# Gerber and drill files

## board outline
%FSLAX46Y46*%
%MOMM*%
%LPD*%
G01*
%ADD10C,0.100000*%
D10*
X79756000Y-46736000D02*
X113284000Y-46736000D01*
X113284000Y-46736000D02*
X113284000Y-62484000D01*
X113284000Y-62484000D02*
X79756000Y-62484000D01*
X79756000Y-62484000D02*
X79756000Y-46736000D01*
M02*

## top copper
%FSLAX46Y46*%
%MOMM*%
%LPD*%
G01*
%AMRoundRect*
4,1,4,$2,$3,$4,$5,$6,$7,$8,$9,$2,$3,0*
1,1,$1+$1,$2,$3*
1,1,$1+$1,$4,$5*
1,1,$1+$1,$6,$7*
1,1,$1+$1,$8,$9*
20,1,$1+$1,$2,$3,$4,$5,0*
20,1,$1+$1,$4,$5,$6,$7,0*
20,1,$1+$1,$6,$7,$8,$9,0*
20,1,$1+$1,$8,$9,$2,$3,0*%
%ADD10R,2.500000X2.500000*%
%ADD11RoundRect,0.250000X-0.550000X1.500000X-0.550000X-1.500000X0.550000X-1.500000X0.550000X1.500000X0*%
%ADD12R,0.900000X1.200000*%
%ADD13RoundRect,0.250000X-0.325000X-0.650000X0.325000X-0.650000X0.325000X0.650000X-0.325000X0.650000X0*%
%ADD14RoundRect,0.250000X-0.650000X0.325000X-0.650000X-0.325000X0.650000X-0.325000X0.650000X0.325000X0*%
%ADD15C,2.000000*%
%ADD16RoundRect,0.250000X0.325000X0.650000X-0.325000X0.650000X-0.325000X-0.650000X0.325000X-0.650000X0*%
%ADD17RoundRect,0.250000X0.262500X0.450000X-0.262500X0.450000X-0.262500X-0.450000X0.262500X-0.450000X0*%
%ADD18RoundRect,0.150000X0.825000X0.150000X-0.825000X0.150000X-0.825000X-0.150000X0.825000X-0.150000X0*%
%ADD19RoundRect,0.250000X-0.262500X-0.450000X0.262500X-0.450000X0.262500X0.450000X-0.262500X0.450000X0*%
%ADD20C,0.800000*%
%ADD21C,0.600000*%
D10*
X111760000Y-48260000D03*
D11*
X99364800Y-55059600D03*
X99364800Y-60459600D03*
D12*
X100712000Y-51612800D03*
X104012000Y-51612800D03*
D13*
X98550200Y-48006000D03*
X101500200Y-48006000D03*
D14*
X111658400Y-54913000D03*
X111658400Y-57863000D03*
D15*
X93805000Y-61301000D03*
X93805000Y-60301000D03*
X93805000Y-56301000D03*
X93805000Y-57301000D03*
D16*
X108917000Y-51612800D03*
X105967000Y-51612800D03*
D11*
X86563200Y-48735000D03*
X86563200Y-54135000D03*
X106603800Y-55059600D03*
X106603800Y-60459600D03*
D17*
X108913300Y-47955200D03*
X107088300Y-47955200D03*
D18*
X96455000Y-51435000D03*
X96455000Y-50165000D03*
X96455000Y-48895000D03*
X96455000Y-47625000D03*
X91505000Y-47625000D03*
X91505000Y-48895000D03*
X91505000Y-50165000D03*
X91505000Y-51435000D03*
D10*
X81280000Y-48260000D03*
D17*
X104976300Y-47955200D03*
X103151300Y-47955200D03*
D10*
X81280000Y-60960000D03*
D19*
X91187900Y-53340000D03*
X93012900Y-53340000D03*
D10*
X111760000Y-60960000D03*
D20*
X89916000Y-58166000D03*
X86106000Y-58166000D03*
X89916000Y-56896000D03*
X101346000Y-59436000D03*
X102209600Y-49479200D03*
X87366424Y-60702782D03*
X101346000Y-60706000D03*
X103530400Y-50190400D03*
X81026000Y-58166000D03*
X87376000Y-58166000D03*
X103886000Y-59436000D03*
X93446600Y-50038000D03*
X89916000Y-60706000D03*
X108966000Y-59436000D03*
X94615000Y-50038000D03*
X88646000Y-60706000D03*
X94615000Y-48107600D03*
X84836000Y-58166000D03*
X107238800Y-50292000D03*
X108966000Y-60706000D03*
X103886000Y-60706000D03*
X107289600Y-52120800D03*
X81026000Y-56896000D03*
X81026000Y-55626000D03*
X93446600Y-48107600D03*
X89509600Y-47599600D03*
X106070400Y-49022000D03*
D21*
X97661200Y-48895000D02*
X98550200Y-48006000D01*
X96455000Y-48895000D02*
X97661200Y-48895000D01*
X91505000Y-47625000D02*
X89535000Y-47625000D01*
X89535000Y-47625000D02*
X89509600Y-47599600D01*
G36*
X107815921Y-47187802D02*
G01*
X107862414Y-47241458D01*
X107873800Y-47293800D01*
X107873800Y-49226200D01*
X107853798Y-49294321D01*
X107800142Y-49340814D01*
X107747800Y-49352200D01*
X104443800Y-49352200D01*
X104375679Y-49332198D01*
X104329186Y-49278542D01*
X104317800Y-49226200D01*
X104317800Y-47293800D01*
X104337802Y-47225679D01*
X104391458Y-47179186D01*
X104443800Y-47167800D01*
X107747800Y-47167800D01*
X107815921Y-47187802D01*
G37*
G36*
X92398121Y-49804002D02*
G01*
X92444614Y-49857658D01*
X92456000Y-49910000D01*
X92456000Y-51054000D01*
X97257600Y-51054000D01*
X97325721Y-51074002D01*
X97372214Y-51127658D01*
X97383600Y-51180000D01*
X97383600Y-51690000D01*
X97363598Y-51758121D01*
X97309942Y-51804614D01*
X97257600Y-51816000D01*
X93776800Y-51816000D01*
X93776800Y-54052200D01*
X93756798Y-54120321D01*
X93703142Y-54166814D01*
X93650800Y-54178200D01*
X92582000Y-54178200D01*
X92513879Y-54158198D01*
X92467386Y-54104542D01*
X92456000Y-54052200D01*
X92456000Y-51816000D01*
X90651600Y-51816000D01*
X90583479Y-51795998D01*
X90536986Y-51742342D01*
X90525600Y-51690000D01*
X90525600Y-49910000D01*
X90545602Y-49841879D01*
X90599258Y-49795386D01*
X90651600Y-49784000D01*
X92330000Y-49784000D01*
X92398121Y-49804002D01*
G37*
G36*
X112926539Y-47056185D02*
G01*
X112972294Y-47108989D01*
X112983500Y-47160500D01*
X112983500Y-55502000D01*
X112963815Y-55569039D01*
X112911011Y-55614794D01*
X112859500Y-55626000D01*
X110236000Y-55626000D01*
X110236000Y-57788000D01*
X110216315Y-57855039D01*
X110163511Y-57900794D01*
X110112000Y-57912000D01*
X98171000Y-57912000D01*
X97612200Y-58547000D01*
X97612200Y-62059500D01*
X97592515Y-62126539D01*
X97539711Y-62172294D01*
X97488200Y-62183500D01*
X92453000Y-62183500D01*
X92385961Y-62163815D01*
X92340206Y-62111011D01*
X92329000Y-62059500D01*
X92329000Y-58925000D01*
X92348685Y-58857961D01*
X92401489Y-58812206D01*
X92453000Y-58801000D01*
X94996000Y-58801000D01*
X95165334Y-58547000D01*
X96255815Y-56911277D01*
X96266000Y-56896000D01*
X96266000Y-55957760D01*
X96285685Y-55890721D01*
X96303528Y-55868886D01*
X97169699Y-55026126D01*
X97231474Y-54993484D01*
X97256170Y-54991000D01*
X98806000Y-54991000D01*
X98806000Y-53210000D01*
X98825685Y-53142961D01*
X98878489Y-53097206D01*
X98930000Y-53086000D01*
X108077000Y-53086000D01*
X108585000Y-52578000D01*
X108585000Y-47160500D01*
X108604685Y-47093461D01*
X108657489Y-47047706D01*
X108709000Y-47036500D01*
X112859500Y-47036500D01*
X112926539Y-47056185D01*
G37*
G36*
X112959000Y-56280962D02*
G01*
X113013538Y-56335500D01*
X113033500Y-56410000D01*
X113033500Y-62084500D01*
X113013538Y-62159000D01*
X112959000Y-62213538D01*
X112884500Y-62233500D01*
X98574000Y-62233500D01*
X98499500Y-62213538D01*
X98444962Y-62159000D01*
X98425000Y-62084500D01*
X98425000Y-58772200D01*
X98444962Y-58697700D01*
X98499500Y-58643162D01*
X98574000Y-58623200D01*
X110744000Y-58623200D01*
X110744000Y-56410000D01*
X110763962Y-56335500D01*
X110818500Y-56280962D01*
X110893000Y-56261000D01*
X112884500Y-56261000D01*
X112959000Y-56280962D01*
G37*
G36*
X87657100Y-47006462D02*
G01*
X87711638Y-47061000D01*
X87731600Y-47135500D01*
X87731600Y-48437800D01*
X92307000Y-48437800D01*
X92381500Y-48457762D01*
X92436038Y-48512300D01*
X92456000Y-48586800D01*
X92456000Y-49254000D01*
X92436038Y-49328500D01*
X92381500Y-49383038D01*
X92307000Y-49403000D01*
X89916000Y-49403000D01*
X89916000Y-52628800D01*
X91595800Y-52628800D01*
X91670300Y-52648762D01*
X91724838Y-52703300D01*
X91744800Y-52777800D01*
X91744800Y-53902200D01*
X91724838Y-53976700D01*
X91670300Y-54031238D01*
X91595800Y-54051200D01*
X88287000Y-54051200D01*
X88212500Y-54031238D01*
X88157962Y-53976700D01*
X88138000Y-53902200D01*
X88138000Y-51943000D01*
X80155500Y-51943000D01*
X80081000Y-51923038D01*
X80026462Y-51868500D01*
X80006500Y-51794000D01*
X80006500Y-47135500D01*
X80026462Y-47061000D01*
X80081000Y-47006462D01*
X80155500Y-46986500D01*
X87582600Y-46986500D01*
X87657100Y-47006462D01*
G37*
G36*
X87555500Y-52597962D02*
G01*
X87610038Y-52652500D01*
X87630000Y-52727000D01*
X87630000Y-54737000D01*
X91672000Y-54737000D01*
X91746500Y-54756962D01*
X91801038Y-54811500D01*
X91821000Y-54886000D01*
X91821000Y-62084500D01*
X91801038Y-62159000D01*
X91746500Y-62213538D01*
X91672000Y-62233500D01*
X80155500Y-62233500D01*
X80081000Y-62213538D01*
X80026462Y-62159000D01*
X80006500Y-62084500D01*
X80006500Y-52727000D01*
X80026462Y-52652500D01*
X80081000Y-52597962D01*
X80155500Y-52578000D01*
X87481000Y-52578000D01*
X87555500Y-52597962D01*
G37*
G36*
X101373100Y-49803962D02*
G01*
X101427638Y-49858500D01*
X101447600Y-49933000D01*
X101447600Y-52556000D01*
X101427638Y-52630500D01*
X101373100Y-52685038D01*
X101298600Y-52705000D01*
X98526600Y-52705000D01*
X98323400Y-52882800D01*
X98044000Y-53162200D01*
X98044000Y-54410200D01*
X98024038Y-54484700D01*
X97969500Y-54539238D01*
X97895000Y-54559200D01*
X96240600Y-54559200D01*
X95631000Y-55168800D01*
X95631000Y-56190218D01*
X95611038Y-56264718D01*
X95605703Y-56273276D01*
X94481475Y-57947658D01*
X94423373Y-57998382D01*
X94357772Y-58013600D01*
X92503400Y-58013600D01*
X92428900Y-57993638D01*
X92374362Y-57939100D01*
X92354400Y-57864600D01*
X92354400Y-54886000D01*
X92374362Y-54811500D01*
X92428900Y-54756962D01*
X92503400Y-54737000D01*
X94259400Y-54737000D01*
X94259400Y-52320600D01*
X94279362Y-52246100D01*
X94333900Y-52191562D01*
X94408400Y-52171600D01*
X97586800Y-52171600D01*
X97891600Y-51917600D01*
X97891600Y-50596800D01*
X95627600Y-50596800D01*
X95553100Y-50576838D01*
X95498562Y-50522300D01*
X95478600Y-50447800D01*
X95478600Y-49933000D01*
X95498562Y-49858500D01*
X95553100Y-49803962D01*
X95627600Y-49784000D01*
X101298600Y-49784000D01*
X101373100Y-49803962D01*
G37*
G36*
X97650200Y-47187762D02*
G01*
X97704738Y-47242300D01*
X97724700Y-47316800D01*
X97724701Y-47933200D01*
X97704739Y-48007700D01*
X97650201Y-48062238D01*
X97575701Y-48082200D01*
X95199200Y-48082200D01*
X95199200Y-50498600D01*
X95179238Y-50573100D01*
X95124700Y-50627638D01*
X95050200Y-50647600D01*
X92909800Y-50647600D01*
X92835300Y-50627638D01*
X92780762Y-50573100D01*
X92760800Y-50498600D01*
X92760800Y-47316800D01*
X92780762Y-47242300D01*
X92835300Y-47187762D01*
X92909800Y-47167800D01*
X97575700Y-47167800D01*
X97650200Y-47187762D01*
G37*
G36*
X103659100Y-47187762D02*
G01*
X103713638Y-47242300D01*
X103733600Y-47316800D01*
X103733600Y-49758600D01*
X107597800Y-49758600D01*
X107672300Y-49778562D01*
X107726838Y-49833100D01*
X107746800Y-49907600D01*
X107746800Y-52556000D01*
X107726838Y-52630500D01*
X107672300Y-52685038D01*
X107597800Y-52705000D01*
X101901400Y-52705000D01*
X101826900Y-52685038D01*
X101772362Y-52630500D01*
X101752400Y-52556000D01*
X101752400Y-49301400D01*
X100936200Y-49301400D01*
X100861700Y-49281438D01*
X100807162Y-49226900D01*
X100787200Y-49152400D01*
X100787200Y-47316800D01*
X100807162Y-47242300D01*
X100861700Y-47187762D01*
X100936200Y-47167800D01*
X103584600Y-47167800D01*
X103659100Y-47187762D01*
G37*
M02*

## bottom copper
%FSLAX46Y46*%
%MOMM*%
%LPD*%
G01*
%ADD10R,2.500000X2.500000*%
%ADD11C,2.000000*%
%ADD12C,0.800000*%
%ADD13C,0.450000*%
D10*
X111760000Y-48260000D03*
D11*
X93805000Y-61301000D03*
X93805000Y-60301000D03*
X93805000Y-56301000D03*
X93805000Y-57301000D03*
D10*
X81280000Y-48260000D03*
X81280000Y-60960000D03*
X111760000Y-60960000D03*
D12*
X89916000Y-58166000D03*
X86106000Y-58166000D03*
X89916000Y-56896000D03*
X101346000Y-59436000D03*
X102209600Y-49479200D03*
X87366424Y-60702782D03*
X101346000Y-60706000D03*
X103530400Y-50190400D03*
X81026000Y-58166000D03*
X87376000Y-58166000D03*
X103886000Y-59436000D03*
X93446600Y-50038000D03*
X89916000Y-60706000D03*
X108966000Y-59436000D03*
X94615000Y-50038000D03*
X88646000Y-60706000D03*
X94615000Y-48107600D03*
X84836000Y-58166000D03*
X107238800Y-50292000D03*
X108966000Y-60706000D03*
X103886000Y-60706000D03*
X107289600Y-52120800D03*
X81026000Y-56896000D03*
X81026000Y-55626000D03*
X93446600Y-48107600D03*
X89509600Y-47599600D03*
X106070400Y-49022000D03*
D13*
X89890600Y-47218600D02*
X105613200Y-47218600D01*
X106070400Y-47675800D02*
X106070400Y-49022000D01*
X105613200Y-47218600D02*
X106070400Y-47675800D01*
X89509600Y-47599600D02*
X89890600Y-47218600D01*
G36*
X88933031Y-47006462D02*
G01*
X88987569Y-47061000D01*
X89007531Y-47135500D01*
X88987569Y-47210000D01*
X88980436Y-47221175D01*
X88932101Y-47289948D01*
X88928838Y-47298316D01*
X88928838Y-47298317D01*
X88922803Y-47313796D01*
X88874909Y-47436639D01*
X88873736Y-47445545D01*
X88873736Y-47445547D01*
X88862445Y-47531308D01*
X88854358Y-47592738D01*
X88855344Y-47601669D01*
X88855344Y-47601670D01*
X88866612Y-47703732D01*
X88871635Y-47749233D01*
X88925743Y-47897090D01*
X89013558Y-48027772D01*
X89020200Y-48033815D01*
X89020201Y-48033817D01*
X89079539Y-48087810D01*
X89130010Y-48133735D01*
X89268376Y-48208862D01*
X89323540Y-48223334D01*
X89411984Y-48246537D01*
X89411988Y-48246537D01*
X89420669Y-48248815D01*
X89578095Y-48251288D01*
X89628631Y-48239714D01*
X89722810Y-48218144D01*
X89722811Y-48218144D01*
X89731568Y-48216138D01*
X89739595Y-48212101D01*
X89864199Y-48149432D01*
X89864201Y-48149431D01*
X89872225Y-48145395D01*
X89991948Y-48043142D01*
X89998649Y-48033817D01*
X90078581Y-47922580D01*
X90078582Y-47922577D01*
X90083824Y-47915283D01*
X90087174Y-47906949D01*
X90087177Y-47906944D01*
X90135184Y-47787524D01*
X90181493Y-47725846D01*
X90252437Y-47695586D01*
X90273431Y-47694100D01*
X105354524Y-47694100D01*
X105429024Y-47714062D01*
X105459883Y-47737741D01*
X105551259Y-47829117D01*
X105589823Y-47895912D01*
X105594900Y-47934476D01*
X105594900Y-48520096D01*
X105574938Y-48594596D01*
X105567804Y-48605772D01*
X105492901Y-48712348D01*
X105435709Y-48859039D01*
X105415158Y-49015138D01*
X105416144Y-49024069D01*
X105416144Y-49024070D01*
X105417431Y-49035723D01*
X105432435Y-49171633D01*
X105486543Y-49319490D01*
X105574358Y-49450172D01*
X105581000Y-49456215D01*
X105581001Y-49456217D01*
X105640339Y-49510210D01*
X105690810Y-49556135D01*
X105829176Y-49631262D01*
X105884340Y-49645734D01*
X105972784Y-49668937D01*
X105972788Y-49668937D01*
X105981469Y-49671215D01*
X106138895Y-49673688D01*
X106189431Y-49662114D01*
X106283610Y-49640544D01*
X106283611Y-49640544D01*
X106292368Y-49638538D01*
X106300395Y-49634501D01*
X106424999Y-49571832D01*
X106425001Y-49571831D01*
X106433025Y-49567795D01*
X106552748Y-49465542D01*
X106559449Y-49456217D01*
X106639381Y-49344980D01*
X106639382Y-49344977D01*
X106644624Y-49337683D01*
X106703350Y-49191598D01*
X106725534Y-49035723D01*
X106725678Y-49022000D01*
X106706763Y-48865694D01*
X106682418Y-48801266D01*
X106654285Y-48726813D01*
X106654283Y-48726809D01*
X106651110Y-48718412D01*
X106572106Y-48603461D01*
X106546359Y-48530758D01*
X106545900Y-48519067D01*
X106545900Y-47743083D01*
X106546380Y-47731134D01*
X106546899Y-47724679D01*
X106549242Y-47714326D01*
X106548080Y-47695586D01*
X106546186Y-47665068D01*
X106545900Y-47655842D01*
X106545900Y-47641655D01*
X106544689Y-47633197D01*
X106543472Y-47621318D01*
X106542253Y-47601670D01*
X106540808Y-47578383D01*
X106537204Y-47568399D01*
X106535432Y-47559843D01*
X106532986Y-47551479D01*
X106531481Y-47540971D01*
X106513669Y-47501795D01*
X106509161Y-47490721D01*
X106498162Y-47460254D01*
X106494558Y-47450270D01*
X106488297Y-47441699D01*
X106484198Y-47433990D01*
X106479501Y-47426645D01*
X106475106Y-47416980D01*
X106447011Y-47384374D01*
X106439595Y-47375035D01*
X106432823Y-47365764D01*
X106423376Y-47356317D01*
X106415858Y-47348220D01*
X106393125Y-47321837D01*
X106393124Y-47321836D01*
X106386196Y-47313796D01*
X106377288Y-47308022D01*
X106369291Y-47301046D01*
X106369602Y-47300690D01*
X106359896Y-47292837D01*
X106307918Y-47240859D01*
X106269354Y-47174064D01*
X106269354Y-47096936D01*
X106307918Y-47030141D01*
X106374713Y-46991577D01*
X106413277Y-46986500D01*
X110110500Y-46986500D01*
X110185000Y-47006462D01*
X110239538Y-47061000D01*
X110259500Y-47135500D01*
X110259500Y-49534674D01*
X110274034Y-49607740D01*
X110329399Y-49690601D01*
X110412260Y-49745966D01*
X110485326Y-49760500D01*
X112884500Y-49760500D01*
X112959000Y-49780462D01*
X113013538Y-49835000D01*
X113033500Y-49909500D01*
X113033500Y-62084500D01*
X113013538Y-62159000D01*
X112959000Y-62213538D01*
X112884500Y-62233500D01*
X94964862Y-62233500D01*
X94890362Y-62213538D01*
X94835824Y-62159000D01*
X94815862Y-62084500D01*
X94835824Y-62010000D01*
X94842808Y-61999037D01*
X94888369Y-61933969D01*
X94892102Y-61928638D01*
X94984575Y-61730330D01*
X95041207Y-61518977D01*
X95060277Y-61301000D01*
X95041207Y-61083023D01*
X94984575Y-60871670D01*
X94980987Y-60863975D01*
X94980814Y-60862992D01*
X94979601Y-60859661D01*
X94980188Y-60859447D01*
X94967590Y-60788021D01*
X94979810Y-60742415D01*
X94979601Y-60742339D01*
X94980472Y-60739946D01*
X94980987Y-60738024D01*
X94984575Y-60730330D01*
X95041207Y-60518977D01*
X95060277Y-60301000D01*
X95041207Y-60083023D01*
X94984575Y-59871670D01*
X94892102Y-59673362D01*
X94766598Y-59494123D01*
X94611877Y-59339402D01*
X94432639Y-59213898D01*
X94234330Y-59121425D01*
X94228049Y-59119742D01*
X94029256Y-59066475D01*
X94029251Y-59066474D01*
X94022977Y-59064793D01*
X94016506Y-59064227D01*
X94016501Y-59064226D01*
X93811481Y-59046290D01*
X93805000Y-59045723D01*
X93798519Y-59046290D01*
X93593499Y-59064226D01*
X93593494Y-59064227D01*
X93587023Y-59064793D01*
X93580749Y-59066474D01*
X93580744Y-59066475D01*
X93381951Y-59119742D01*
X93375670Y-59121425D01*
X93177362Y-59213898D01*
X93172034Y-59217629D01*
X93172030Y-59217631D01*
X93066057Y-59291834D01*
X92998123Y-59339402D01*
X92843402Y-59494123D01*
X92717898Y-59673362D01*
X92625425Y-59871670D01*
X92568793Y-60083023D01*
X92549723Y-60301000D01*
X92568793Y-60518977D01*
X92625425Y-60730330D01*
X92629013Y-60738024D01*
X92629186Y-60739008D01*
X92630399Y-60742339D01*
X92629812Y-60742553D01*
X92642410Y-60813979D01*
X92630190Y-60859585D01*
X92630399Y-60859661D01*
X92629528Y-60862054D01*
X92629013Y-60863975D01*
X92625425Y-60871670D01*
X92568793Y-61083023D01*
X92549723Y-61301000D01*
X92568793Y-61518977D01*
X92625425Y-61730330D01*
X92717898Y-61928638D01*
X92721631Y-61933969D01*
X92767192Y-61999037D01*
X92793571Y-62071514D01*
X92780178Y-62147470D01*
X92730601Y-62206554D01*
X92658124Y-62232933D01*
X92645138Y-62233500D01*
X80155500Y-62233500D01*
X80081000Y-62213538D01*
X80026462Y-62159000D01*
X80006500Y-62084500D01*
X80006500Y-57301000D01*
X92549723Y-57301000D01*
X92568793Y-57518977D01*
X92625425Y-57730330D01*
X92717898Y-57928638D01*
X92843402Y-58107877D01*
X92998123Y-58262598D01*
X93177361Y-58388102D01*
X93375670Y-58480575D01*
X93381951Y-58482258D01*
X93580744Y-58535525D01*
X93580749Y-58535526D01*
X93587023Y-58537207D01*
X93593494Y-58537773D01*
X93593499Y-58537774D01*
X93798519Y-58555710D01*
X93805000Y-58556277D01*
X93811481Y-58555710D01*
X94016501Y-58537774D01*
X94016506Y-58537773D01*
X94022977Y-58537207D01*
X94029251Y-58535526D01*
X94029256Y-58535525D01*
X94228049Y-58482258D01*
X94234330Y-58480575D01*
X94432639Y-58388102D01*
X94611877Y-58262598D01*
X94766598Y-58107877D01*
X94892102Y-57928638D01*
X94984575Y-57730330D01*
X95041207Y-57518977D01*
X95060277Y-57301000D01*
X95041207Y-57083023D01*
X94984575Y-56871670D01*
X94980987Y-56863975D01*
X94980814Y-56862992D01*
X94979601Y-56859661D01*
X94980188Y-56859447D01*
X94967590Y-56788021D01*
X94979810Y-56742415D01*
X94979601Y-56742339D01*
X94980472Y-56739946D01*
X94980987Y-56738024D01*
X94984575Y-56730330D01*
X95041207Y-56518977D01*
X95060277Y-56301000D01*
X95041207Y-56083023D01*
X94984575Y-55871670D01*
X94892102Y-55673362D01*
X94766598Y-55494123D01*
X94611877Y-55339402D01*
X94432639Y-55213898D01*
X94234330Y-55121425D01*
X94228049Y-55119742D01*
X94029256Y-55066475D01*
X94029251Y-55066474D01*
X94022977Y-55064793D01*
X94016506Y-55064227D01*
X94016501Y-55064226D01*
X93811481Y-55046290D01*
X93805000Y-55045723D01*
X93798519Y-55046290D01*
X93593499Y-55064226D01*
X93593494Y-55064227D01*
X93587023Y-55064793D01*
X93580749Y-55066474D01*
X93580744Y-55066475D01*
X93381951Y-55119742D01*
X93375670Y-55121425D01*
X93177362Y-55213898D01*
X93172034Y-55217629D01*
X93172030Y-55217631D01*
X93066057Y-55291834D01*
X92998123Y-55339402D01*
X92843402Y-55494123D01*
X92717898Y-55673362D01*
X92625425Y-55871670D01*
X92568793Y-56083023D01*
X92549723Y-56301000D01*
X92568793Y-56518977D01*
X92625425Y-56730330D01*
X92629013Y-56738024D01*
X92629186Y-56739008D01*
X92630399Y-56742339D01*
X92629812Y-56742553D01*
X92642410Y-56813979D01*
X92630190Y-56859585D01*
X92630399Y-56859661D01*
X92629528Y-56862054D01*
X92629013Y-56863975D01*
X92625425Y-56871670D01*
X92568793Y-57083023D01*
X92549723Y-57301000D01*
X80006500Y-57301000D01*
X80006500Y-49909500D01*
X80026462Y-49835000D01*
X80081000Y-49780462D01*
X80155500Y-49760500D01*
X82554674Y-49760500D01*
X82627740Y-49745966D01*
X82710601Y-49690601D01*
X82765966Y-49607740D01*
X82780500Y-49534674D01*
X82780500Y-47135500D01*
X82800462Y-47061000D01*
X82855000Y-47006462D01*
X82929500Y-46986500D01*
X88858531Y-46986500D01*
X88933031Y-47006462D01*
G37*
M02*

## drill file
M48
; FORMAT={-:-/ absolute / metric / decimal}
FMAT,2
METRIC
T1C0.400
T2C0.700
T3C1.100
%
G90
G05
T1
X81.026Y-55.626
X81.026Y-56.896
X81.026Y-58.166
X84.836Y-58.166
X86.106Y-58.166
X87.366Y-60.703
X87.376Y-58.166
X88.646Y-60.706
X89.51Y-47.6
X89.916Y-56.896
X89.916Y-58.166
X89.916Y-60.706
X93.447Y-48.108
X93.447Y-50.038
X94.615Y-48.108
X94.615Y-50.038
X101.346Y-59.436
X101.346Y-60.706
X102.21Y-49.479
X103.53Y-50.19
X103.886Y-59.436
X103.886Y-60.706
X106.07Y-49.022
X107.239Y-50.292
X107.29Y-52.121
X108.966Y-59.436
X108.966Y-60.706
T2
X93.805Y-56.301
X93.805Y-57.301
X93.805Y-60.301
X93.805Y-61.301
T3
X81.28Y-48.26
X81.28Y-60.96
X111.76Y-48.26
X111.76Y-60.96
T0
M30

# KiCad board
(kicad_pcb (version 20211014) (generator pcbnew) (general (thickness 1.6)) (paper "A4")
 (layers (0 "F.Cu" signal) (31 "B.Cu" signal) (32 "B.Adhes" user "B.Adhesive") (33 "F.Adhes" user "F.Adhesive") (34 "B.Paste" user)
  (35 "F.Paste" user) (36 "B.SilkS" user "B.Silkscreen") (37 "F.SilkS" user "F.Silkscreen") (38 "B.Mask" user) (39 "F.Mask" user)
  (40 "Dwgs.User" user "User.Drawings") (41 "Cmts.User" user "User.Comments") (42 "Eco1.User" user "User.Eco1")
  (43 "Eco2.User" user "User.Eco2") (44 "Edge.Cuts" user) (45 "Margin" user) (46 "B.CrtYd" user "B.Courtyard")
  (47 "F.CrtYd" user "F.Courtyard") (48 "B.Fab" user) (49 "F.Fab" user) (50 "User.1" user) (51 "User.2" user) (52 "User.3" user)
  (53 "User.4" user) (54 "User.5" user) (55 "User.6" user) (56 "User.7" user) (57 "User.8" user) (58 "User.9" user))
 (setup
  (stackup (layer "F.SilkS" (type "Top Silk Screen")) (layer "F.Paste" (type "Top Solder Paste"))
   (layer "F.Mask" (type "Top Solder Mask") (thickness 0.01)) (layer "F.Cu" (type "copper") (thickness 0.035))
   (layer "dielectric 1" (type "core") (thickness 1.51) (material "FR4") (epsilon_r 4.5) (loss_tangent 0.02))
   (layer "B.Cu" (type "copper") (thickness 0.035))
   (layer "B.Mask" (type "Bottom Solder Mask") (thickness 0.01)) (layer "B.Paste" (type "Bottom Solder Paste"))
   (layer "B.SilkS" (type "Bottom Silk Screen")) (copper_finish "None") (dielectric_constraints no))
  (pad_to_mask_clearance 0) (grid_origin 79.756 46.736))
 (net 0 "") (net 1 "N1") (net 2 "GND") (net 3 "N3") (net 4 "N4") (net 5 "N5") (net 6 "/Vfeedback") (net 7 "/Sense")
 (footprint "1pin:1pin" (layer "F.Cu") (at 111.76 48.26)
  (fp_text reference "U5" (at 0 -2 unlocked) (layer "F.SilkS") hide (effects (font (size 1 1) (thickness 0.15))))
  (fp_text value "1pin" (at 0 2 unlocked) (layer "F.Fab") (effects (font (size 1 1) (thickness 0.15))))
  (pad "1" thru_hole rect (at 0 0) (size 2.5 2.5) (drill 1.1) (layers *.Cu *.Mask) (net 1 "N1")))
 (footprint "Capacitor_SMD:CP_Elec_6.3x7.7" (layer "F.Cu") (at 99.3648 57.7596 -90)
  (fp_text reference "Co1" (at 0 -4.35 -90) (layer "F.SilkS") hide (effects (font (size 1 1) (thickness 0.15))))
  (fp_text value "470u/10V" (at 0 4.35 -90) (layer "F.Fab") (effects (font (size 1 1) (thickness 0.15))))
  (pad "1" smd roundrect (at -2.7 0 270) (size 3.5 1.6) (layers "F.Cu" "F.Paste" "F.Mask") (roundrect_rratio 0.15625) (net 1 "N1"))
  (pad "2" smd roundrect (at 2.7 0 270) (size 3.5 1.6) (layers "F.Cu" "F.Paste" "F.Mask") (roundrect_rratio 0.15625) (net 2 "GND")))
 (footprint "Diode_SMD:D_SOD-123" (layer "F.Cu") (at 102.362 51.6128)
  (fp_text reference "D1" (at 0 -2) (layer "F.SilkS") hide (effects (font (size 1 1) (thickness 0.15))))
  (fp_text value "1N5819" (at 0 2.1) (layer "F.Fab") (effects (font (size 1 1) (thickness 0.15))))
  (pad "1" smd rect (at -1.65 0) (size 0.9 1.2) (layers "F.Cu" "F.Paste" "F.Mask") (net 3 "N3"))
  (pad "2" smd rect (at 1.65 0) (size 0.9 1.2) (layers "F.Cu" "F.Paste" "F.Mask") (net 2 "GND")))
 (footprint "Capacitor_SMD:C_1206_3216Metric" (layer "F.Cu") (at 100.0252 48.006)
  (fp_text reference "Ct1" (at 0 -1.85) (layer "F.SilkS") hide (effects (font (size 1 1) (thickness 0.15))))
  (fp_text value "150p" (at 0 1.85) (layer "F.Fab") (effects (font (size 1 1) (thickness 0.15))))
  (pad "1" smd roundrect (at -1.475 0) (size 1.15 1.8) (layers "F.Cu" "F.Paste" "F.Mask") (roundrect_rratio 0.2173913043) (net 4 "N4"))
  (pad "2" smd roundrect (at 1.475 0) (size 1.15 1.8) (layers "F.Cu" "F.Paste" "F.Mask") (roundrect_rratio 0.2173913043) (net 2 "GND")))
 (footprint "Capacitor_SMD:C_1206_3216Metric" (layer "F.Cu") (at 111.6584 56.388 -90)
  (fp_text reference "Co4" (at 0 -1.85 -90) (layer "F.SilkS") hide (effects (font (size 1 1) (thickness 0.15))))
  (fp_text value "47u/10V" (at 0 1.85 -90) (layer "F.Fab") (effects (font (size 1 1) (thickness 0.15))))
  (pad "1" smd roundrect (at -1.475 0 270) (size 1.15 1.8) (layers "F.Cu" "F.Paste" "F.Mask") (roundrect_rratio 0.2173913043) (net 1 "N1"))
  (pad "2" smd roundrect (at 1.475 0 270) (size 1.15 1.8) (layers "F.Cu" "F.Paste" "F.Mask") (roundrect_rratio 0.2173913043) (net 2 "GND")))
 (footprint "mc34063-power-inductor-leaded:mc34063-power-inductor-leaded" (layer "F.Cu") (at 93.805 58.801)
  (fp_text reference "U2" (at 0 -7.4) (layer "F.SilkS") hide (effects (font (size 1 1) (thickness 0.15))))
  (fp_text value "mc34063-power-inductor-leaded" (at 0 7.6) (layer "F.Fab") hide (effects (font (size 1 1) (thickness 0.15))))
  (pad "1" thru_hole circle (at 0 2.5 180) (size 2 2) (drill 0.7) (layers *.Cu *.Mask) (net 1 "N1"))
  (pad "1" thru_hole circle (at 0 1.5 180) (size 2 2) (drill 0.7) (layers *.Cu *.Mask) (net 1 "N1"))
  (pad "2" thru_hole circle (at 0 -2.5 180) (size 2 2) (drill 0.7) (layers *.Cu *.Mask) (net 3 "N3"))
  (pad "2" thru_hole circle (at 0 -1.5 180) (size 2 2) (drill 0.7) (layers *.Cu *.Mask) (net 3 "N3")))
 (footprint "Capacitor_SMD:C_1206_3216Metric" (layer "F.Cu") (at 107.442 51.6128 180)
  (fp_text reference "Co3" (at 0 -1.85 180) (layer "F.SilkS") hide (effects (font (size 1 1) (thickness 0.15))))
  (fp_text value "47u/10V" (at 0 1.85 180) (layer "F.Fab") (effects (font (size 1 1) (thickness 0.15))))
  (pad "1" smd roundrect (at -1.475 0 180) (size 1.15 1.8) (layers "F.Cu" "F.Paste" "F.Mask") (roundrect_rratio 0.2173913043) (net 1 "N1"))
  (pad "2" smd roundrect (at 1.475 0 180) (size 1.15 1.8) (layers "F.Cu" "F.Paste" "F.Mask") (roundrect_rratio 0.2173913043) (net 2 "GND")))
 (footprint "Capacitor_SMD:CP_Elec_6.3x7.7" (layer "F.Cu") (at 86.5632 51.435 -90)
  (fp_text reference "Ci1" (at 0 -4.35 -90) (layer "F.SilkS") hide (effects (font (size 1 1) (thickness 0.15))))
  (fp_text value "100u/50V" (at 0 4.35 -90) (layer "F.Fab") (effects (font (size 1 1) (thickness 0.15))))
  (pad "1" smd roundrect (at -2.7 0 270) (size 3.5 1.6) (layers "F.Cu" "F.Paste" "F.Mask") (roundrect_rratio 0.15625) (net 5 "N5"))
  (pad "2" smd roundrect (at 2.7 0 270) (size 3.5 1.6) (layers "F.Cu" "F.Paste" "F.Mask") (roundrect_rratio 0.15625) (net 2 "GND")))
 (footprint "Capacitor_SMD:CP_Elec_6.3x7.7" (layer "F.Cu") (at 106.6038 57.7596 -90)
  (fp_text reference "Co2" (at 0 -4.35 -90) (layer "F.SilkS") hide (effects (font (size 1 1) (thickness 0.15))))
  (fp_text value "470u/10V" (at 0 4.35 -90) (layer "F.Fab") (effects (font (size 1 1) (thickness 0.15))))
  (pad "1" smd roundrect (at -2.7 0 270) (size 3.5 1.6) (layers "F.Cu" "F.Paste" "F.Mask") (roundrect_rratio 0.15625) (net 1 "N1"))
  (pad "2" smd roundrect (at 2.7 0 270) (size 3.5 1.6) (layers "F.Cu" "F.Paste" "F.Mask") (roundrect_rratio 0.15625) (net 2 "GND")))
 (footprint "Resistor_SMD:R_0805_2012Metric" (layer "F.Cu") (at 108.0008 47.9552 180)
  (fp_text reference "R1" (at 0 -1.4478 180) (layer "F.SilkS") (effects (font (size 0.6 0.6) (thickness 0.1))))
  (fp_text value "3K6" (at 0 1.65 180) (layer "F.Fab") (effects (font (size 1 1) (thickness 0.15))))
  (pad "1" smd roundrect (at -0.9125 0 180) (size 1.025 1.4) (layers "F.Cu" "F.Paste" "F.Mask") (roundrect_rratio 0.243902439) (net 1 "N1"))
  (pad "2" smd roundrect (at 0.9125 0 180) (size 1.025 1.4) (layers "F.Cu" "F.Paste" "F.Mask") (roundrect_rratio 0.243902439)
   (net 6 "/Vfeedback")))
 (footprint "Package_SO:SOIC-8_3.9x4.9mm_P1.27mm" (layer "F.Cu") (at 93.98 49.53 180)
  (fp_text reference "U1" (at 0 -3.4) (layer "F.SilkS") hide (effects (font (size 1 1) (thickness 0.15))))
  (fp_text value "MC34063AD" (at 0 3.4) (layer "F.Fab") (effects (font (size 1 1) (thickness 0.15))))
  (pad "1" smd roundrect (at -2.475 -1.905 180) (size 1.95 0.6) (layers "F.Cu" "F.Paste" "F.Mask") (roundrect_rratio 0.25) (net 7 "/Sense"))
  (pad "2" smd roundrect (at -2.475 -0.635 180) (size 1.95 0.6) (layers "F.Cu" "F.Paste" "F.Mask") (roundrect_rratio 0.25) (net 3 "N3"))
  (pad "3" smd roundrect (at -2.475 0.635 180) (size 1.95 0.6) (layers "F.Cu" "F.Paste" "F.Mask") (roundrect_rratio 0.25) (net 4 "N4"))
  (pad "4" smd roundrect (at -2.475 1.905 180) (size 1.95 0.6) (layers "F.Cu" "F.Paste" "F.Mask") (roundrect_rratio 0.25) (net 2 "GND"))
  (pad "5" smd roundrect (at 2.475 1.905 180) (size 1.95 0.6) (layers "F.Cu" "F.Paste" "F.Mask") (roundrect_rratio 0.25)
   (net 6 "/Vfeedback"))
  (pad "6" smd roundrect (at 2.475 0.635 180) (size 1.95 0.6) (layers "F.Cu" "F.Paste" "F.Mask") (roundrect_rratio 0.25) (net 5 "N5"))
  (pad "7" smd roundrect (at 2.475 -0.635 180) (size 1.95 0.6) (layers "F.Cu" "F.Paste" "F.Mask") (roundrect_rratio 0.25) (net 7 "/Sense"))
  (pad "8" smd roundrect (at 2.475 -1.905 180) (size 1.95 0.6) (layers "F.Cu" "F.Paste" "F.Mask") (roundrect_rratio 0.25) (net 7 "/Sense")))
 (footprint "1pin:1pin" (layer "F.Cu") (at 81.28 48.26)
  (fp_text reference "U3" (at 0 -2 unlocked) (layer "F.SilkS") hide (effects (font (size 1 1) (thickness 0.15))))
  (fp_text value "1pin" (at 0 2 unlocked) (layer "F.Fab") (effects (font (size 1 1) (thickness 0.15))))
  (pad "1" thru_hole rect (at 0 0) (size 2.5 2.5) (drill 1.1) (layers *.Cu *.Mask) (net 5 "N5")))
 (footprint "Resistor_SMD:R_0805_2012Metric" (layer "F.Cu") (at 104.0638 47.9552 180)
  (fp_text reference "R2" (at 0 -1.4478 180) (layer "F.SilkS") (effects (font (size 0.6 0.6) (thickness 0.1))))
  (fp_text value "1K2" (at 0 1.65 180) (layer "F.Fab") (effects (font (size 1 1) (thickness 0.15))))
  (pad "1" smd roundrect (at -0.9125 0 180) (size 1.025 1.4) (layers "F.Cu" "F.Paste" "F.Mask") (roundrect_rratio 0.243902439)
   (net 6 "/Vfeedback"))
  (pad "2" smd roundrect (at 0.9125 0 180) (size 1.025 1.4) (layers "F.Cu" "F.Paste" "F.Mask") (roundrect_rratio 0.243902439) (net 2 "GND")))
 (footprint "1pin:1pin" (layer "F.Cu") (at 81.28 60.96)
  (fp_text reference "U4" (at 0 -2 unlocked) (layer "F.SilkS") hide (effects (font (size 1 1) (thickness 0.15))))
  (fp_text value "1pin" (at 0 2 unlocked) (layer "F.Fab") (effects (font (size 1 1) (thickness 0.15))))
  (pad "1" thru_hole rect (at 0 0) (size 2.5 2.5) (drill 1.1) (layers *.Cu *.Mask) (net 2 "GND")))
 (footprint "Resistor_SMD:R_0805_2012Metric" (layer "F.Cu") (at 92.1004 53.34)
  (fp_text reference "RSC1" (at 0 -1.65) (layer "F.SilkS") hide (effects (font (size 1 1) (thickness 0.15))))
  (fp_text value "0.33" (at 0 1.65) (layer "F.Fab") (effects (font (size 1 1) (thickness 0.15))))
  (pad "1" smd roundrect (at -0.9125 0) (size 1.025 1.4) (layers "F.Cu" "F.Paste" "F.Mask") (roundrect_rratio 0.243902439) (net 5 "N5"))
  (pad "2" smd roundrect (at 0.9125 0) (size 1.025 1.4) (layers "F.Cu" "F.Paste" "F.Mask") (roundrect_rratio 0.243902439) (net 7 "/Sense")))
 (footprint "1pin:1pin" (layer "F.Cu") (at 111.76 60.96)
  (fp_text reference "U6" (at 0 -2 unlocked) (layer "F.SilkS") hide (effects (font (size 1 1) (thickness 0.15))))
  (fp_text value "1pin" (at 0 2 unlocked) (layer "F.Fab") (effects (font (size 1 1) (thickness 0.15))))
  (pad "1" thru_hole rect (at 0 0) (size 2.5 2.5) (drill 1.1) (layers *.Cu *.Mask) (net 2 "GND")))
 (gr_rect (start 79.756 46.736) (end 113.284 62.484) (layer "Edge.Cuts") (width 0.1) (fill none))
 (via (at 89.916 58.166) (size 0.8) (drill 0.4) (layers "F.Cu" "B.Cu") (free) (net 2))
 (via (at 86.106 58.166) (size 0.8) (drill 0.4) (layers "F.Cu" "B.Cu") (free) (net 2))
 (via (at 89.916 56.896) (size 0.8) (drill 0.4) (layers "F.Cu" "B.Cu") (free) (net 2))
 (via (at 101.346 59.436) (size 0.8) (drill 0.4) (layers "F.Cu" "B.Cu") (free) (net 2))
 (via (at 102.2096 49.4792) (size 0.8) (drill 0.4) (layers "F.Cu" "B.Cu") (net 2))
 (via (at 87.366424 60.702782) (size 0.8) (drill 0.4) (layers "F.Cu" "B.Cu") (free) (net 2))
 (via (at 101.346 60.706) (size 0.8) (drill 0.4) (layers "F.Cu" "B.Cu") (free) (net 2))
 (via (at 103.5304 50.1904) (size 0.8) (drill 0.4) (layers "F.Cu" "B.Cu") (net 2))
 (via (at 81.026 58.166) (size 0.8) (drill 0.4) (layers "F.Cu" "B.Cu") (free) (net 2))
 (via (at 87.376 58.166) (size 0.8) (drill 0.4) (layers "F.Cu" "B.Cu") (free) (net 2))
 (via (at 103.886 59.436) (size 0.8) (drill 0.4) (layers "F.Cu" "B.Cu") (free) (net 2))
 (via (at 93.4466 50.038) (size 0.8) (drill 0.4) (layers "F.Cu" "B.Cu") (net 2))
 (via (at 89.916 60.706) (size 0.8) (drill 0.4) (layers "F.Cu" "B.Cu") (free) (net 2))
 (via (at 108.966 59.436) (size 0.8) (drill 0.4) (layers "F.Cu" "B.Cu") (free) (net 2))
 (via (at 94.615 50.038) (size 0.8) (drill 0.4) (layers "F.Cu" "B.Cu") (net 2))
 (via (at 88.646 60.706) (size 0.8) (drill 0.4) (layers "F.Cu" "B.Cu") (free) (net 2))
 (via (at 94.615 48.1076) (size 0.8) (drill 0.4) (layers "F.Cu" "B.Cu") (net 2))
 (via (at 84.836 58.166) (size 0.8) (drill 0.4) (layers "F.Cu" "B.Cu") (free) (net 2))
 (via (at 107.2388 50.292) (size 0.8) (drill 0.4) (layers "F.Cu" "B.Cu") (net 2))
 (via (at 108.966 60.706) (size 0.8) (drill 0.4) (layers "F.Cu" "B.Cu") (free) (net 2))
 (via (at 103.886 60.706) (size 0.8) (drill 0.4) (layers "F.Cu" "B.Cu") (free) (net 2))
 (via (at 107.2896 52.1208) (size 0.8) (drill 0.4) (layers "F.Cu" "B.Cu") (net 2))
 (via (at 81.026 56.896) (size 0.8) (drill 0.4) (layers "F.Cu" "B.Cu") (free) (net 2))
 (via (at 81.026 55.626) (size 0.8) (drill 0.4) (layers "F.Cu" "B.Cu") (free) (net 2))
 (via (at 93.4466 48.1076) (size 0.8) (drill 0.4) (layers "F.Cu" "B.Cu") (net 2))
 (segment (start 97.6612 48.895) (end 98.5502 48.006) (width 0.6) (layer "F.Cu") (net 4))
 (segment (start 96.455 48.895) (end 97.6612 48.895) (width 0.6) (layer "F.Cu") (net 4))
 (segment (start 91.505 47.625) (end 89.535 47.625) (width 0.6) (layer "F.Cu") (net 6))
 (segment (start 89.535 47.625) (end 89.5096 47.5996) (width 0.6) (layer "F.Cu") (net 6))
 (via (at 89.5096 47.5996) (size 0.8) (drill 0.4) (layers "F.Cu" "B.Cu") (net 6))
 (via (at 106.0704 49.022) (size 0.8) (drill 0.4) (layers "F.Cu" "B.Cu") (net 6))
 (segment (start 89.8906 47.2186) (end 105.6132 47.2186) (width 0.45) (layer "B.Cu") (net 6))
 (segment (start 106.0704 47.6758) (end 106.0704 49.022) (width 0.45) (layer "B.Cu") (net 6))
 (segment (start 105.6132 47.2186) (end 106.0704 47.6758) (width 0.45) (layer "B.Cu") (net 6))
 (segment (start 89.5096 47.5996) (end 89.8906 47.2186) (width 0.45) (layer "B.Cu") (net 6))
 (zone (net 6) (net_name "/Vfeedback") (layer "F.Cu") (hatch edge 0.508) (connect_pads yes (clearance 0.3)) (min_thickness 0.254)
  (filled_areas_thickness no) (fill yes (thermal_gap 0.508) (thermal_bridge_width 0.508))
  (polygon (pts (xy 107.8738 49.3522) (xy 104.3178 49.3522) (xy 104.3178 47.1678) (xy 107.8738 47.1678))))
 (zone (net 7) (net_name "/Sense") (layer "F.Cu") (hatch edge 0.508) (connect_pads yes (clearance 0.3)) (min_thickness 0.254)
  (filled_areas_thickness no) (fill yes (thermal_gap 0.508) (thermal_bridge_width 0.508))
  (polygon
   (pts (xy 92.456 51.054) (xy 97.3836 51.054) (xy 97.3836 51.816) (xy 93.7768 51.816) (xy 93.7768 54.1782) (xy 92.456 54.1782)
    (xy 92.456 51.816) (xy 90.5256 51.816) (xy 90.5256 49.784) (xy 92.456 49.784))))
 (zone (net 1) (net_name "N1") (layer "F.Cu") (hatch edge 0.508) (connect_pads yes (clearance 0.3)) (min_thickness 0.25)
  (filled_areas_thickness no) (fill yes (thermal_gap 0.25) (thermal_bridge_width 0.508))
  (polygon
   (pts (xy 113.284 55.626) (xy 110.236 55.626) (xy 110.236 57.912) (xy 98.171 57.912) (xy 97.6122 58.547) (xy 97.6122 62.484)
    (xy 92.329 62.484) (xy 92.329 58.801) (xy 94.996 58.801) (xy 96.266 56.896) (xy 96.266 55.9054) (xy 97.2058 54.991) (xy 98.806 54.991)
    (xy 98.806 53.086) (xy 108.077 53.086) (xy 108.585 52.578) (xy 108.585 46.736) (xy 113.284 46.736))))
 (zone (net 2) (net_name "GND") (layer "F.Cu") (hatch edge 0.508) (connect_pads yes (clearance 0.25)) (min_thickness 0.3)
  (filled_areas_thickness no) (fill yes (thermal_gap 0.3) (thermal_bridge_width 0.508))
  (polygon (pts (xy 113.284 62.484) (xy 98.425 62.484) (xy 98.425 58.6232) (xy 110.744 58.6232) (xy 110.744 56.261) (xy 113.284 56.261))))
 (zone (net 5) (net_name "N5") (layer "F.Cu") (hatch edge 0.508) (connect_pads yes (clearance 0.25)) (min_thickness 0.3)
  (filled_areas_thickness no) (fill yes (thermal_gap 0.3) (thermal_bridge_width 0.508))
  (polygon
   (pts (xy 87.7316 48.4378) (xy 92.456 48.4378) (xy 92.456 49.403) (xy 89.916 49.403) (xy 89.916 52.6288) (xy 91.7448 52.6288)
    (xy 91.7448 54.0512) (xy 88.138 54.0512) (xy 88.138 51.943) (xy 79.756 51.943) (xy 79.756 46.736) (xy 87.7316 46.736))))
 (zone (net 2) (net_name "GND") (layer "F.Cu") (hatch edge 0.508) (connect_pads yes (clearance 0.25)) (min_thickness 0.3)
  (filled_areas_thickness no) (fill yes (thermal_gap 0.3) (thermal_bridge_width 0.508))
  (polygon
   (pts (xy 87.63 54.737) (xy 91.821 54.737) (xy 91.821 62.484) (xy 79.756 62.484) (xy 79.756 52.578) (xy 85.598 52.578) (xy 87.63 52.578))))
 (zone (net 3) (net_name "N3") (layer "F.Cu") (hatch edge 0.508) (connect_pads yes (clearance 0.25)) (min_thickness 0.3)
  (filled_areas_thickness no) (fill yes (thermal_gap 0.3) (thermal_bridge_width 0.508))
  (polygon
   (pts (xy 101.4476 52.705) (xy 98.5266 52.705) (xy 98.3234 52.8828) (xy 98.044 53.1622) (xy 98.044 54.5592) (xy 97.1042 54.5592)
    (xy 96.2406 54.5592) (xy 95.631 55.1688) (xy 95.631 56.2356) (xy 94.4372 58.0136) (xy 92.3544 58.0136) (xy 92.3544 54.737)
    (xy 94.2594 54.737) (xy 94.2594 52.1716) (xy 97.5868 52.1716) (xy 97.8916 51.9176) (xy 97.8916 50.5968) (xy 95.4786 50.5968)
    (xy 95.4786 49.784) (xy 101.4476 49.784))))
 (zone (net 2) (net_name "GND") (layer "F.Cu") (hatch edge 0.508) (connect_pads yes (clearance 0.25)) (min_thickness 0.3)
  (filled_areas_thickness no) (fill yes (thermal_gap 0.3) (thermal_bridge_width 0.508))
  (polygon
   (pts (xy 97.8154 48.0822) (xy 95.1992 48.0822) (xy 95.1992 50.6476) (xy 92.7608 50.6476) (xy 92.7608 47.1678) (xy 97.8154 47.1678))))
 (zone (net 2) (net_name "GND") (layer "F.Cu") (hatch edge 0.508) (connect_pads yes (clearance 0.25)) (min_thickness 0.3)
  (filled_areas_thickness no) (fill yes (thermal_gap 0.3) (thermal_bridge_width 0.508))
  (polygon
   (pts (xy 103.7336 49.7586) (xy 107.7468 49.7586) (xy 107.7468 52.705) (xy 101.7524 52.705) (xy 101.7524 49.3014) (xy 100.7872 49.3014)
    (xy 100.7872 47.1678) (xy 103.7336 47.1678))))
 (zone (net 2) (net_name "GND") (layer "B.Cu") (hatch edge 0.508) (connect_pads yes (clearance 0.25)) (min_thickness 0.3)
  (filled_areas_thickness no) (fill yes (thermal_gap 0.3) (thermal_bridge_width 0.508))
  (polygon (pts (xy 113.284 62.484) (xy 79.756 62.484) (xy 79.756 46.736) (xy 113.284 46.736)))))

